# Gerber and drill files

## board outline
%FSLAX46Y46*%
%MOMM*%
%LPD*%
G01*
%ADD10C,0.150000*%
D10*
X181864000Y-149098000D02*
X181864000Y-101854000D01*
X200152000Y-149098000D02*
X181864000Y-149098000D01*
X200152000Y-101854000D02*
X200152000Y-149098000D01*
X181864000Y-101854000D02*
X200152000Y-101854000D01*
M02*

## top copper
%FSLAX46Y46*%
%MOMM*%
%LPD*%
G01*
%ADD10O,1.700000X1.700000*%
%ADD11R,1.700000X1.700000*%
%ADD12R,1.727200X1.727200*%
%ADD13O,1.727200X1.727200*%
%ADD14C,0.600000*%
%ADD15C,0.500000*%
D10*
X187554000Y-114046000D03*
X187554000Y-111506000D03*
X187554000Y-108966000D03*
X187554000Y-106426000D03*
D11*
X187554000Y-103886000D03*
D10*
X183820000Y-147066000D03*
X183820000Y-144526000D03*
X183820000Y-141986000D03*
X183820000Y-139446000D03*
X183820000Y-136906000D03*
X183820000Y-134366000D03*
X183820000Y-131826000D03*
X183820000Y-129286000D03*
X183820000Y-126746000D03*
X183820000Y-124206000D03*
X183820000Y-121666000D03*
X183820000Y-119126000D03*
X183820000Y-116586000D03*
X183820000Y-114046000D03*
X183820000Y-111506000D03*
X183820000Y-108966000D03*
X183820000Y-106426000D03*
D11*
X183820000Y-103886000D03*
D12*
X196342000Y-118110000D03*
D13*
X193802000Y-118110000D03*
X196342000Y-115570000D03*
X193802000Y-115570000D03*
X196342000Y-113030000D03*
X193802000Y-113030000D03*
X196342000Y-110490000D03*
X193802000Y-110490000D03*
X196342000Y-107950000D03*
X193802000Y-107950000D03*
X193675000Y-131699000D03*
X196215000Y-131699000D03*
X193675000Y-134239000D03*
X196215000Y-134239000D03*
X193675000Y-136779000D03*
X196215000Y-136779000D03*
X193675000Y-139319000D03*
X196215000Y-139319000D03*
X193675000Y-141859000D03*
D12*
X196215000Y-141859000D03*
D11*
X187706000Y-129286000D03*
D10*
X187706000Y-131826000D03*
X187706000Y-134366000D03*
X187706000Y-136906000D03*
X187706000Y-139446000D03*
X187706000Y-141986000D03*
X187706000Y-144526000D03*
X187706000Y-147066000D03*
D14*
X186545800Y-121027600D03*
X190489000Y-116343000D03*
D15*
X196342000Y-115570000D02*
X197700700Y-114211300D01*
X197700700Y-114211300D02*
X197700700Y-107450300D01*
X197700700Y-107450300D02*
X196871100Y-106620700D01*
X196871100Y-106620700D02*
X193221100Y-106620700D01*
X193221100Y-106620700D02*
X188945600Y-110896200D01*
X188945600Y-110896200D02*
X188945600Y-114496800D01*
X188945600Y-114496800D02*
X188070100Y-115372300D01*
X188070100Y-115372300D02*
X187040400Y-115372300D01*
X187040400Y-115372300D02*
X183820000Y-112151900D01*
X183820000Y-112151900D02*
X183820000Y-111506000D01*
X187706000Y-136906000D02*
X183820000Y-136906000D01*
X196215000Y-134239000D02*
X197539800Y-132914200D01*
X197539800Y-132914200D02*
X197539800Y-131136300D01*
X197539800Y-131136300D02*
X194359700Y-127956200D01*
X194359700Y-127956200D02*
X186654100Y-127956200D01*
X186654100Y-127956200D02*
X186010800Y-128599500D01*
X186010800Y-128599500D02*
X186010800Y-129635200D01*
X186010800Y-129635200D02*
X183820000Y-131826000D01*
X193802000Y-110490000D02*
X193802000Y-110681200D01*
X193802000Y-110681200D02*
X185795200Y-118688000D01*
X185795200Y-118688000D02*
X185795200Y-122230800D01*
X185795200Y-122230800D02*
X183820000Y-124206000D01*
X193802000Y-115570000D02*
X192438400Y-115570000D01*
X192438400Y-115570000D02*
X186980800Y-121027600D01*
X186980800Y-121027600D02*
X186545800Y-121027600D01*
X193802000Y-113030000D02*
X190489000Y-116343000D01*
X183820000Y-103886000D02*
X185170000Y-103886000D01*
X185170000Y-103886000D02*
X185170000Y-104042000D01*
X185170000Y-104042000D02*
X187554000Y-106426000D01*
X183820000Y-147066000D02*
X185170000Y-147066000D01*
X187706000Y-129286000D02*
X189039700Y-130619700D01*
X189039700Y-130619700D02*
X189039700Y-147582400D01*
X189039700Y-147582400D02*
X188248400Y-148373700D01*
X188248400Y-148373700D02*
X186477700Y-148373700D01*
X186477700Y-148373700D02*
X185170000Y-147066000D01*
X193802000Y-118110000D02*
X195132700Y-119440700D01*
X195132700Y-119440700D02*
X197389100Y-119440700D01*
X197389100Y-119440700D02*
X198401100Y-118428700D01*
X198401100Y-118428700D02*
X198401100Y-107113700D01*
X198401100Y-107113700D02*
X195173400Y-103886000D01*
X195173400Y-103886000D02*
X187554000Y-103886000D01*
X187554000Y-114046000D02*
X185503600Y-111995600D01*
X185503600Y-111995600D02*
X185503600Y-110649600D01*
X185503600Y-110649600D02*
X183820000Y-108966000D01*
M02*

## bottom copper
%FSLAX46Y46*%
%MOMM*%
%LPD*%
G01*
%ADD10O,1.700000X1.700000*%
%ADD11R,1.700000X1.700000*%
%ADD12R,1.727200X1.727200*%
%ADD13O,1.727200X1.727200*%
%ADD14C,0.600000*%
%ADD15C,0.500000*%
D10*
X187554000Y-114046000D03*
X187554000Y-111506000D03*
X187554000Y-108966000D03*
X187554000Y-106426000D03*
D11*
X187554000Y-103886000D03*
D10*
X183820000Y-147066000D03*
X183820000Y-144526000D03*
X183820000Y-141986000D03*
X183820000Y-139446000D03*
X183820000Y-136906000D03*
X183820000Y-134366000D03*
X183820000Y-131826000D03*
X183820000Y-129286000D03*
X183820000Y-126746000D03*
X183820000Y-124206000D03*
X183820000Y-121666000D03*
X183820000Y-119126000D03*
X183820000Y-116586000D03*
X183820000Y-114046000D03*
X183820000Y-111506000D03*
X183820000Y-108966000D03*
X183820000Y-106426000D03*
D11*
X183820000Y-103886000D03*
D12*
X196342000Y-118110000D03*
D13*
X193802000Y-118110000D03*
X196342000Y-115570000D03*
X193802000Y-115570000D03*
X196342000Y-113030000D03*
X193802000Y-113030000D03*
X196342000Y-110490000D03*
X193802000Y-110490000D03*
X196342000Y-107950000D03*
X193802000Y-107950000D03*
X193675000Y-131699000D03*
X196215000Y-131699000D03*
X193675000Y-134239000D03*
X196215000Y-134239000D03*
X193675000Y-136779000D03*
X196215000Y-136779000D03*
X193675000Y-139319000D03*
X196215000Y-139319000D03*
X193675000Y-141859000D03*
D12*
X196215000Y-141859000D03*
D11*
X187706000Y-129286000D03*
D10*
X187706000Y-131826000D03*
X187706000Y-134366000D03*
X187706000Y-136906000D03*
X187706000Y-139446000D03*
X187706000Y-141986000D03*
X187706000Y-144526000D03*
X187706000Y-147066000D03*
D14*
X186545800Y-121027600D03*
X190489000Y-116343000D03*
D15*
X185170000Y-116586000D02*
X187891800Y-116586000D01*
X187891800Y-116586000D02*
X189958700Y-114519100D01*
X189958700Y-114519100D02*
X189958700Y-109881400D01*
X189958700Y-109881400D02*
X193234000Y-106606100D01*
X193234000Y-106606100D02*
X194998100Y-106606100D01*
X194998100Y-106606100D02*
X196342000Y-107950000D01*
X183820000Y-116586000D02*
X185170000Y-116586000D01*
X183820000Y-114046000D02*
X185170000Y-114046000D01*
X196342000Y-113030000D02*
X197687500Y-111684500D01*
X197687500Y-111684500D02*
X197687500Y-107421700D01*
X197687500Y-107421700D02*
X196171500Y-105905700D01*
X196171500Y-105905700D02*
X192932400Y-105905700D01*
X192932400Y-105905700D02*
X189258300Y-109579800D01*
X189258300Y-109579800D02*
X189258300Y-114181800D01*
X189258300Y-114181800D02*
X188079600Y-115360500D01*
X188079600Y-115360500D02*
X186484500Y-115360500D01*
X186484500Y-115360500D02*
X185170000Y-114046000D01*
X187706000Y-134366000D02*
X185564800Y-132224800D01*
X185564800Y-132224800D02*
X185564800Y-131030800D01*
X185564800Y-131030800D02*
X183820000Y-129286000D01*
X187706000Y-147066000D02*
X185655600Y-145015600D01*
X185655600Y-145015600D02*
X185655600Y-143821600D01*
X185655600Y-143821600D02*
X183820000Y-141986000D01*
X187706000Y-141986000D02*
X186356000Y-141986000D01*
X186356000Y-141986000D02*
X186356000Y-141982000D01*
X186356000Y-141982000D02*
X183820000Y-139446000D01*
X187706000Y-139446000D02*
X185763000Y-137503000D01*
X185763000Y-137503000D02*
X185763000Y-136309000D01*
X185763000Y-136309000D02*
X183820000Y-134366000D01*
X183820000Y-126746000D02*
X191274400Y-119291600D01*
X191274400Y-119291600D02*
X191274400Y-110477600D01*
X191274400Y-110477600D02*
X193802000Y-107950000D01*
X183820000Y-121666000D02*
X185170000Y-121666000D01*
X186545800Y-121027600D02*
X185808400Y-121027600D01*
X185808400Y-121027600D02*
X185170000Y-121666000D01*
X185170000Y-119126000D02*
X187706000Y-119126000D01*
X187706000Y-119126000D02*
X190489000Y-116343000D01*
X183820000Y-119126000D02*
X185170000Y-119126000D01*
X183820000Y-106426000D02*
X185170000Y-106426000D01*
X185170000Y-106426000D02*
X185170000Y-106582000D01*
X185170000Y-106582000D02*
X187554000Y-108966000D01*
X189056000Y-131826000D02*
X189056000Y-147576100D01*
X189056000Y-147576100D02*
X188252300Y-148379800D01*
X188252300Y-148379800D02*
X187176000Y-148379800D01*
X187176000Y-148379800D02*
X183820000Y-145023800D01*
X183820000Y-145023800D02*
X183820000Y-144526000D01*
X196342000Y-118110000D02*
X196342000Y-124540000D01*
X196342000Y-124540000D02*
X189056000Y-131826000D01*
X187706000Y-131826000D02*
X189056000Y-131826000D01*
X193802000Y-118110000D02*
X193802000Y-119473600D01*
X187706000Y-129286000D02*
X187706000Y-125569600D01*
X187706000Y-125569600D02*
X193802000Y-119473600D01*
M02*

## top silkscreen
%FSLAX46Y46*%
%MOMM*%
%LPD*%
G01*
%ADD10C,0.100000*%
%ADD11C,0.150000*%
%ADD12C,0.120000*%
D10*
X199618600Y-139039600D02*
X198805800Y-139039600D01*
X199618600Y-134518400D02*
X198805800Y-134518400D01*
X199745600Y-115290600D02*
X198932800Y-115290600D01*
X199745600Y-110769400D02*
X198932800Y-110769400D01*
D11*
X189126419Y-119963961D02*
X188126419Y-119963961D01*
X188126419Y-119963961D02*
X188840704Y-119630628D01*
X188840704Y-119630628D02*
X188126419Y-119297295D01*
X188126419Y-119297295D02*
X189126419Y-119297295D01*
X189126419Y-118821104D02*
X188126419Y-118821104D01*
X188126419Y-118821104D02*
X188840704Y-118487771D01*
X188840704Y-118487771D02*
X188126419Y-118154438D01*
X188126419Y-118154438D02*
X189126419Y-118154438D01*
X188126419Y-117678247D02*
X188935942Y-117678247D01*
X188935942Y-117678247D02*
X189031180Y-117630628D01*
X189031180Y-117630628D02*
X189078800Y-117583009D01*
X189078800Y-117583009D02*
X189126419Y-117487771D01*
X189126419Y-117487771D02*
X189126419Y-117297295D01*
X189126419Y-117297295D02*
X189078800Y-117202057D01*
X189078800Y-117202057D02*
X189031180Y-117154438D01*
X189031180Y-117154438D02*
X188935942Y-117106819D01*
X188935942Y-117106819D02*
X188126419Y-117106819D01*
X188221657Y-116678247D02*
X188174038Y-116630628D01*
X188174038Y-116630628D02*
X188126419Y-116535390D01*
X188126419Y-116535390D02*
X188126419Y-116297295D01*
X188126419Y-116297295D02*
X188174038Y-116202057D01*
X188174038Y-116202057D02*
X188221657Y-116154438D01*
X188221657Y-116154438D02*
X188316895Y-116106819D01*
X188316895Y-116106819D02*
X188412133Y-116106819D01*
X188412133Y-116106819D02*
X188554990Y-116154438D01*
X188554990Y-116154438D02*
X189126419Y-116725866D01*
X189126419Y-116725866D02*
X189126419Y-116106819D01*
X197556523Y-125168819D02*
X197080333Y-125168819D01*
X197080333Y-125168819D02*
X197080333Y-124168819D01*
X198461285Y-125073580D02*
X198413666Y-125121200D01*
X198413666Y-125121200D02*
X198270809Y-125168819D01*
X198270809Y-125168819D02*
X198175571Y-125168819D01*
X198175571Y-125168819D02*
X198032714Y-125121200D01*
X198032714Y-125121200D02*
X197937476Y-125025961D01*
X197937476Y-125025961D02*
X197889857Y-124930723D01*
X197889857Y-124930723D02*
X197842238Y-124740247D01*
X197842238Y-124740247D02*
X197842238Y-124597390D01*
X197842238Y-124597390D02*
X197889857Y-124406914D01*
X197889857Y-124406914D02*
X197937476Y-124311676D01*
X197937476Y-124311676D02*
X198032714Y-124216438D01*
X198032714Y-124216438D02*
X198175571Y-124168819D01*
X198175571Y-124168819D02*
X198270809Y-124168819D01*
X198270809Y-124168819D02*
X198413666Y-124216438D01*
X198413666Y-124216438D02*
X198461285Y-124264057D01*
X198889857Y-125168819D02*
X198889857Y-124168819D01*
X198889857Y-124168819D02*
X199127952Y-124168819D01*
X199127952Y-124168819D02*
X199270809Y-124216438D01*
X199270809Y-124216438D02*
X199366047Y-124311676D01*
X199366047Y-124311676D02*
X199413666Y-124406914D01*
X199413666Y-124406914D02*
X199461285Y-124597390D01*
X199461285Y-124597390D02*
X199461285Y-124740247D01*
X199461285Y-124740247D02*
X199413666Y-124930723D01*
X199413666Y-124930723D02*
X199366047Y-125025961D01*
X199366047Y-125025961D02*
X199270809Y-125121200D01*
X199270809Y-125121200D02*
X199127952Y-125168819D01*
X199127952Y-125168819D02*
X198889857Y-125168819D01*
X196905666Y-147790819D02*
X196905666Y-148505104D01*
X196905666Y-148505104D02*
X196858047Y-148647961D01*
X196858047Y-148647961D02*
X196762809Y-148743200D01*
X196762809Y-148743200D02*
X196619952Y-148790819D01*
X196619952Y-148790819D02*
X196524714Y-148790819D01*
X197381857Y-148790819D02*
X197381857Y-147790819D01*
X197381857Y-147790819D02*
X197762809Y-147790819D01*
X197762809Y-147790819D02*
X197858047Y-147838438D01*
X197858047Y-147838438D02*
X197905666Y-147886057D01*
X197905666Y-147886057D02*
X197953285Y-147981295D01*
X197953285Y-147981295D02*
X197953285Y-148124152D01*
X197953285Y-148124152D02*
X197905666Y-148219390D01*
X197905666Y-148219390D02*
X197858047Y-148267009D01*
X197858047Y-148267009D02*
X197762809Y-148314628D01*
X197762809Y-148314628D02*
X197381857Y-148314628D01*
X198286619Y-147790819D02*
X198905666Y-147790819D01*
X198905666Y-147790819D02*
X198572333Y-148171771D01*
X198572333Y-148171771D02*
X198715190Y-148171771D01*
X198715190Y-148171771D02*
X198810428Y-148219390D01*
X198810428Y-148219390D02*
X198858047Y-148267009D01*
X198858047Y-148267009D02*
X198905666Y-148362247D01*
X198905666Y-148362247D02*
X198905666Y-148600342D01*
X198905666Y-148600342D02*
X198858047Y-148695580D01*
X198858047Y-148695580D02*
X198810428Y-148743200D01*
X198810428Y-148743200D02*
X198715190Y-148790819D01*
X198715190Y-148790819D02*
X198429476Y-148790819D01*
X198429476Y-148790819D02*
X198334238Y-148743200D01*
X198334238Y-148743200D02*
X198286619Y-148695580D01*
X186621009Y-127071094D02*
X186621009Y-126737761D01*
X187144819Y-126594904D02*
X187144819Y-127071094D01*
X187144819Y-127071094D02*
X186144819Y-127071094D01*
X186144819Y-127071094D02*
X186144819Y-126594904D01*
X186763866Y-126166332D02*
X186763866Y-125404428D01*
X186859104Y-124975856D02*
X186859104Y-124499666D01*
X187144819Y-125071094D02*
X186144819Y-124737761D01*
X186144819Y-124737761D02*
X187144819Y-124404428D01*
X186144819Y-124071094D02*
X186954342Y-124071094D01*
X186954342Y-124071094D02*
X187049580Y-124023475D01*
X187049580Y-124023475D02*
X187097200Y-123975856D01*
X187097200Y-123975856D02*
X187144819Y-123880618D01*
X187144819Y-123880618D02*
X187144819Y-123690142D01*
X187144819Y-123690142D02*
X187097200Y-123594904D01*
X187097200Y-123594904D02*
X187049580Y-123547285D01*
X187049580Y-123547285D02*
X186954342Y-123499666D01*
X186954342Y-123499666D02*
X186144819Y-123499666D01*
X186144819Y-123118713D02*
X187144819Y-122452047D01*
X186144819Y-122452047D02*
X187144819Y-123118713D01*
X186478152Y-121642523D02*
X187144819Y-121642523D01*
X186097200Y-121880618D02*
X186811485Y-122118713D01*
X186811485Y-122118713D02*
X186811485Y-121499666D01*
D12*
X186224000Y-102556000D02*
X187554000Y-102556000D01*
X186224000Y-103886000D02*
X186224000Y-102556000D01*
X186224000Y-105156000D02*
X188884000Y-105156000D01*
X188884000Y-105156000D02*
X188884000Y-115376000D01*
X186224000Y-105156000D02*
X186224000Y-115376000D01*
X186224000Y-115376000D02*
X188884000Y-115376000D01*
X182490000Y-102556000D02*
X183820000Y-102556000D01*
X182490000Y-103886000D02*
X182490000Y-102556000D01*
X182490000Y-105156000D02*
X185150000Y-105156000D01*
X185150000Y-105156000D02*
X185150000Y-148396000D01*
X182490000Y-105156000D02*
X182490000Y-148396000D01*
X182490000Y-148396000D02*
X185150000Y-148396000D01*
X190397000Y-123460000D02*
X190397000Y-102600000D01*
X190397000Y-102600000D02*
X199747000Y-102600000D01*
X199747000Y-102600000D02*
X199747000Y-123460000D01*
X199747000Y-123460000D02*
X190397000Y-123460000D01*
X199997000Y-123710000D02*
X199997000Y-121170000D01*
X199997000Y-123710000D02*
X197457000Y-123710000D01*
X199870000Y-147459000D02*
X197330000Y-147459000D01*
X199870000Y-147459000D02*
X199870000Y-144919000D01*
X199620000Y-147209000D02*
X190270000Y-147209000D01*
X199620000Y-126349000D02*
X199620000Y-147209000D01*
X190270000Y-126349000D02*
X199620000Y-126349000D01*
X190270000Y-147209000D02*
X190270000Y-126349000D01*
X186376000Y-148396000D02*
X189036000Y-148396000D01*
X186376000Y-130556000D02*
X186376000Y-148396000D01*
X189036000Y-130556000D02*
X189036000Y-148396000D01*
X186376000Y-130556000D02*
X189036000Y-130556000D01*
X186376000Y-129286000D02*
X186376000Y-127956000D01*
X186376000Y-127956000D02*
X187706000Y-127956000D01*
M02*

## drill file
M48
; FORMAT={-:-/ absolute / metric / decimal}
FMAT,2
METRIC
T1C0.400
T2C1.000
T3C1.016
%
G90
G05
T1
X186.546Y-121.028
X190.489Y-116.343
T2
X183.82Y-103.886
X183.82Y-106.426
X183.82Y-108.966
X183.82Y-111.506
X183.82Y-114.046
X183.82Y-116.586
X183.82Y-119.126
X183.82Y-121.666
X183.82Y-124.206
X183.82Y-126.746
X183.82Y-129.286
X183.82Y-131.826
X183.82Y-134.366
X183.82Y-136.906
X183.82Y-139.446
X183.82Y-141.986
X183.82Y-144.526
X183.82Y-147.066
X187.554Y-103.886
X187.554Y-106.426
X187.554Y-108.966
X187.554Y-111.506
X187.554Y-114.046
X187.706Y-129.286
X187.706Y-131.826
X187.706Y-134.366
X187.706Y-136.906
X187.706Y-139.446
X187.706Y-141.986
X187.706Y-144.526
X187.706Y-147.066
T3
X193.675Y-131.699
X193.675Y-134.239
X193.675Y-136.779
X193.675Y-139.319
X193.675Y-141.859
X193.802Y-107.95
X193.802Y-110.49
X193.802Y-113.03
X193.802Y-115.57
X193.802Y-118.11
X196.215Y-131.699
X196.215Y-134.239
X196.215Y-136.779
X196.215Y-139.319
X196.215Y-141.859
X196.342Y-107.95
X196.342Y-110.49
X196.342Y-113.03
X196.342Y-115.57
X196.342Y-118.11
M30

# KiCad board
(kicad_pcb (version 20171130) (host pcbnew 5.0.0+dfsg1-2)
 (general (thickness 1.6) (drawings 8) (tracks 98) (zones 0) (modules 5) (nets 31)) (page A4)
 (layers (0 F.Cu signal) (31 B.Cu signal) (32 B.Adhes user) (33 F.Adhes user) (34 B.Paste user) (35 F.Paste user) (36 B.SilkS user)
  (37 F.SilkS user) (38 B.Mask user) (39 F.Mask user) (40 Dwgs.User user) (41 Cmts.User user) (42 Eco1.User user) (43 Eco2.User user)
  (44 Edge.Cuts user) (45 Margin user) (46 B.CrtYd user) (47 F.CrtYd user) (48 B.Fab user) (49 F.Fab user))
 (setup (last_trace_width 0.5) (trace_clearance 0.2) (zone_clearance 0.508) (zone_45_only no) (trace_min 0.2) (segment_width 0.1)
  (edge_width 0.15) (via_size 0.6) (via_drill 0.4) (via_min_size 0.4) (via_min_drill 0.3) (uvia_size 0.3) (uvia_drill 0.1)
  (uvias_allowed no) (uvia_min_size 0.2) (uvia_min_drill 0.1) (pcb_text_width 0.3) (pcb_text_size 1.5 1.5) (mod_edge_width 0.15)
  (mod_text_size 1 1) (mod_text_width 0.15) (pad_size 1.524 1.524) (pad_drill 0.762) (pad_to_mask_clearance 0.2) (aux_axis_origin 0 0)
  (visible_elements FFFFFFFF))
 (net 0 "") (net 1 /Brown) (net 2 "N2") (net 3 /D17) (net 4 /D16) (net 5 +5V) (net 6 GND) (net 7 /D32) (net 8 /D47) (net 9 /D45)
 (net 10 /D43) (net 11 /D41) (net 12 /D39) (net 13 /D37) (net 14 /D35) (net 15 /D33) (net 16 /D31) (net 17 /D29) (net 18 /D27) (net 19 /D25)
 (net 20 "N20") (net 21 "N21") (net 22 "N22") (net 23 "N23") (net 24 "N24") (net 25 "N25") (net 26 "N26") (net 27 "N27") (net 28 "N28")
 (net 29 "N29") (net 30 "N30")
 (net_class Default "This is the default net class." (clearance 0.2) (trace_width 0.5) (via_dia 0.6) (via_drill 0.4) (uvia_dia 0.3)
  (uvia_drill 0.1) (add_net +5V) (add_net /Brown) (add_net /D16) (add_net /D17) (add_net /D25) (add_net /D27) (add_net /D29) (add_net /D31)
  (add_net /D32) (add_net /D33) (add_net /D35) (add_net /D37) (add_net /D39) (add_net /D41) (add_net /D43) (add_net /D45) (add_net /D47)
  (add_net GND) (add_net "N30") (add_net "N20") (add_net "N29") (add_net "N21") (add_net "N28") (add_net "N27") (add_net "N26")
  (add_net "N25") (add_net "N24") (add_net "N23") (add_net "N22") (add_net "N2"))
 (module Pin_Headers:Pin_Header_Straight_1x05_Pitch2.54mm (layer F.Cu) (at 187.554 103.886)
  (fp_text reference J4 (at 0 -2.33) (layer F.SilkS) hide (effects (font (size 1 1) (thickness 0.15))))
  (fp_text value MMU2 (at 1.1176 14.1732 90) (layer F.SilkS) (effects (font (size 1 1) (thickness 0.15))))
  (fp_line (start -1.33 -1.33) (end 0 -1.33) (layer F.SilkS) (width 0.12))
  (fp_line (start -1.33 0) (end -1.33 -1.33) (layer F.SilkS) (width 0.12))
  (fp_line (start -1.33 1.27) (end 1.33 1.27) (layer F.SilkS) (width 0.12))
  (fp_line (start 1.33 1.27) (end 1.33 11.49) (layer F.SilkS) (width 0.12))
  (fp_line (start -1.33 1.27) (end -1.33 11.49) (layer F.SilkS) (width 0.12))
  (fp_line (start -1.33 11.49) (end 1.33 11.49) (layer F.SilkS) (width 0.12))
  (pad 5 thru_hole oval (at 0 10.16) (size 1.7 1.7) (drill 1) (layers *.Cu *.Mask) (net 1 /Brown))
  (pad 4 thru_hole oval (at 0 7.62) (size 1.7 1.7) (drill 1) (layers *.Cu *.Mask) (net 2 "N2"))
  (pad 3 thru_hole oval (at 0 5.08) (size 1.7 1.7) (drill 1) (layers *.Cu *.Mask) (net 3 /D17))
  (pad 2 thru_hole oval (at 0 2.54) (size 1.7 1.7) (drill 1) (layers *.Cu *.Mask) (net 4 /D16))
  (pad 1 thru_hole rect (at 0 0) (size 1.7 1.7) (drill 1) (layers *.Cu *.Mask) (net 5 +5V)))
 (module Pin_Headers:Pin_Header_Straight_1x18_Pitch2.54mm (layer F.Cu) (at 183.82 103.886)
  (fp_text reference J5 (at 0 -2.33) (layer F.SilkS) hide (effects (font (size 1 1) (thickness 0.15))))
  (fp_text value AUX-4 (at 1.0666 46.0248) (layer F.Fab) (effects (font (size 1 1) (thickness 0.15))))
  (fp_line (start -1.33 -1.33) (end 0 -1.33) (layer F.SilkS) (width 0.12))
  (fp_line (start -1.33 0) (end -1.33 -1.33) (layer F.SilkS) (width 0.12))
  (fp_line (start -1.33 1.27) (end 1.33 1.27) (layer F.SilkS) (width 0.12))
  (fp_line (start 1.33 1.27) (end 1.33 44.51) (layer F.SilkS) (width 0.12))
  (fp_line (start -1.33 1.27) (end -1.33 44.51) (layer F.SilkS) (width 0.12))
  (fp_line (start -1.33 44.51) (end 1.33 44.51) (layer F.SilkS) (width 0.12))
  (pad 18 thru_hole oval (at 0 43.18) (size 1.7 1.7) (drill 1) (layers *.Cu *.Mask) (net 5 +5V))
  (pad 17 thru_hole oval (at 0 40.64) (size 1.7 1.7) (drill 1) (layers *.Cu *.Mask) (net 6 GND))
  (pad 16 thru_hole oval (at 0 38.1) (size 1.7 1.7) (drill 1) (layers *.Cu *.Mask) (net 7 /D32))
  (pad 15 thru_hole oval (at 0 35.56) (size 1.7 1.7) (drill 1) (layers *.Cu *.Mask) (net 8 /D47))
  (pad 14 thru_hole oval (at 0 33.02) (size 1.7 1.7) (drill 1) (layers *.Cu *.Mask) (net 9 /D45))
  (pad 13 thru_hole oval (at 0 30.48) (size 1.7 1.7) (drill 1) (layers *.Cu *.Mask) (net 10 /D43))
  (pad 12 thru_hole oval (at 0 27.94) (size 1.7 1.7) (drill 1) (layers *.Cu *.Mask) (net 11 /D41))
  (pad 11 thru_hole oval (at 0 25.4) (size 1.7 1.7) (drill 1) (layers *.Cu *.Mask) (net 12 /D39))
  (pad 10 thru_hole oval (at 0 22.86) (size 1.7 1.7) (drill 1) (layers *.Cu *.Mask) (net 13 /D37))
  (pad 9 thru_hole oval (at 0 20.32) (size 1.7 1.7) (drill 1) (layers *.Cu *.Mask) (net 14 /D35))
  (pad 8 thru_hole oval (at 0 17.78) (size 1.7 1.7) (drill 1) (layers *.Cu *.Mask) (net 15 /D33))
  (pad 7 thru_hole oval (at 0 15.24) (size 1.7 1.7) (drill 1) (layers *.Cu *.Mask) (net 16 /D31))
  (pad 6 thru_hole oval (at 0 12.7) (size 1.7 1.7) (drill 1) (layers *.Cu *.Mask) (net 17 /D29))
  (pad 5 thru_hole oval (at 0 10.16) (size 1.7 1.7) (drill 1) (layers *.Cu *.Mask) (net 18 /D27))
  (pad 4 thru_hole oval (at 0 7.62) (size 1.7 1.7) (drill 1) (layers *.Cu *.Mask) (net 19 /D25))
  (pad 3 thru_hole oval (at 0 5.08) (size 1.7 1.7) (drill 1) (layers *.Cu *.Mask) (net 1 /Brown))
  (pad 2 thru_hole oval (at 0 2.54) (size 1.7 1.7) (drill 1) (layers *.Cu *.Mask) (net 3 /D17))
  (pad 1 thru_hole rect (at 0 0) (size 1.7 1.7) (drill 1) (layers *.Cu *.Mask) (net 4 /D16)))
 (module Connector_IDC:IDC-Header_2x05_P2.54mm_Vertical (layer F.Cu) (at 196.342 118.11 180)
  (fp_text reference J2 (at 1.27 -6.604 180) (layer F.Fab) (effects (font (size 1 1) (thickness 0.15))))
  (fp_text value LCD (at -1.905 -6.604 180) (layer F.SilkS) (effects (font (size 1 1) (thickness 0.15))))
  (fp_line (start 5.945 -5.35) (end 5.945 15.51) (layer F.SilkS) (width 0.12))
  (fp_line (start 5.945 15.51) (end -3.405 15.51) (layer F.SilkS) (width 0.12))
  (fp_line (start -3.405 15.51) (end -3.405 -5.35) (layer F.SilkS) (width 0.12))
  (fp_line (start -3.405 -5.35) (end 5.945 -5.35) (layer F.SilkS) (width 0.12))
  (fp_line (start -3.655 -5.6) (end -3.655 -3.06) (layer F.SilkS) (width 0.12))
  (fp_line (start -3.655 -5.6) (end -1.115 -5.6) (layer F.SilkS) (width 0.12))
  (pad 1 thru_hole rect (at 0 0 180) (size 1.7272 1.7272) (drill 1.016) (layers *.Cu *.Mask) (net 6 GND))
  (pad 2 thru_hole oval (at 2.54 0 180) (size 1.7272 1.7272) (drill 1.016) (layers *.Cu *.Mask) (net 5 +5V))
  (pad 3 thru_hole oval (at 0 2.54 180) (size 1.7272 1.7272) (drill 1.016) (layers *.Cu *.Mask) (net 19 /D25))
  (pad 4 thru_hole oval (at 2.54 2.54 180) (size 1.7272 1.7272) (drill 1.016) (layers *.Cu *.Mask) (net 15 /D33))
  (pad 5 thru_hole oval (at 0 5.08 180) (size 1.7272 1.7272) (drill 1.016) (layers *.Cu *.Mask) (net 18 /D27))
  (pad 6 thru_hole oval (at 2.54 5.08 180) (size 1.7272 1.7272) (drill 1.016) (layers *.Cu *.Mask) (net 16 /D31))
  (pad 7 thru_hole oval (at 0 7.62 180) (size 1.7272 1.7272) (drill 1.016) (layers *.Cu *.Mask) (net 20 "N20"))
  (pad 8 thru_hole oval (at 2.54 7.62 180) (size 1.7272 1.7272) (drill 1.016) (layers *.Cu *.Mask) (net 14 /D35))
  (pad 9 thru_hole oval (at 0 10.16 180) (size 1.7272 1.7272) (drill 1.016) (layers *.Cu *.Mask) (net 17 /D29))
  (pad 10 thru_hole oval (at 2.54 10.16 180) (size 1.7272 1.7272) (drill 1.016) (layers *.Cu *.Mask) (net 13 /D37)))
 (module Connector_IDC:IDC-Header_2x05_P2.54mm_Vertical (layer F.Cu) (at 196.215 141.859 180)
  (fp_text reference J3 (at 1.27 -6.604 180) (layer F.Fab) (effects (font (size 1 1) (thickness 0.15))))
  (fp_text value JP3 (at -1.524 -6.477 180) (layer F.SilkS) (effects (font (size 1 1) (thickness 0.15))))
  (fp_line (start -3.655 -5.6) (end -1.115 -5.6) (layer F.SilkS) (width 0.12))
  (fp_line (start -3.655 -5.6) (end -3.655 -3.06) (layer F.SilkS) (width 0.12))
  (fp_line (start -3.405 -5.35) (end 5.945 -5.35) (layer F.SilkS) (width 0.12))
  (fp_line (start -3.405 15.51) (end -3.405 -5.35) (layer F.SilkS) (width 0.12))
  (fp_line (start 5.945 15.51) (end -3.405 15.51) (layer F.SilkS) (width 0.12))
  (fp_line (start 5.945 -5.35) (end 5.945 15.51) (layer F.SilkS) (width 0.12))
  (pad 10 thru_hole oval (at 2.54 10.16 180) (size 1.7272 1.7272) (drill 1.016) (layers *.Cu *.Mask) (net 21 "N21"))
  (pad 9 thru_hole oval (at 0 10.16 180) (size 1.7272 1.7272) (drill 1.016) (layers *.Cu *.Mask) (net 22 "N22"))
  (pad 8 thru_hole oval (at 2.54 7.62 180) (size 1.7272 1.7272) (drill 1.016) (layers *.Cu *.Mask) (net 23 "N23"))
  (pad 7 thru_hole oval (at 0 7.62 180) (size 1.7272 1.7272) (drill 1.016) (layers *.Cu *.Mask) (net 11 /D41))
  (pad 6 thru_hole oval (at 2.54 5.08 180) (size 1.7272 1.7272) (drill 1.016) (layers *.Cu *.Mask) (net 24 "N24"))
  (pad 5 thru_hole oval (at 0 5.08 180) (size 1.7272 1.7272) (drill 1.016) (layers *.Cu *.Mask) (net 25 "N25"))
  (pad 4 thru_hole oval (at 2.54 2.54 180) (size 1.7272 1.7272) (drill 1.016) (layers *.Cu *.Mask) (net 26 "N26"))
  (pad 3 thru_hole oval (at 0 2.54 180) (size 1.7272 1.7272) (drill 1.016) (layers *.Cu *.Mask) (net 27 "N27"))
  (pad 2 thru_hole oval (at 2.54 0 180) (size 1.7272 1.7272) (drill 1.016) (layers *.Cu *.Mask) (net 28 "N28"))
  (pad 1 thru_hole rect (at 0 0 180) (size 1.7272 1.7272) (drill 1.016) (layers *.Cu *.Mask) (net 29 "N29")))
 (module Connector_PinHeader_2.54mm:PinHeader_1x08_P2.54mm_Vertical (layer F.Cu) (at 187.706 129.286)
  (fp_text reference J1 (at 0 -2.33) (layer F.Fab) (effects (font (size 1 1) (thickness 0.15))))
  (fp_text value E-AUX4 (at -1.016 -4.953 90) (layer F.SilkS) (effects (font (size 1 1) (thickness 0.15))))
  (fp_line (start -1.33 19.11) (end 1.33 19.11) (layer F.SilkS) (width 0.12))
  (fp_line (start -1.33 1.27) (end -1.33 19.11) (layer F.SilkS) (width 0.12))
  (fp_line (start 1.33 1.27) (end 1.33 19.11) (layer F.SilkS) (width 0.12))
  (fp_line (start -1.33 1.27) (end 1.33 1.27) (layer F.SilkS) (width 0.12))
  (fp_line (start -1.33 0) (end -1.33 -1.33) (layer F.SilkS) (width 0.12))
  (fp_line (start -1.33 -1.33) (end 0 -1.33) (layer F.SilkS) (width 0.12))
  (pad 1 thru_hole rect (at 0 0) (size 1.7 1.7) (drill 1) (layers *.Cu *.Mask) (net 5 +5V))
  (pad 2 thru_hole oval (at 0 2.54) (size 1.7 1.7) (drill 1) (layers *.Cu *.Mask) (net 6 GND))
  (pad 3 thru_hole oval (at 0 5.08) (size 1.7 1.7) (drill 1) (layers *.Cu *.Mask) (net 12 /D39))
  (pad 4 thru_hole oval (at 0 7.62) (size 1.7 1.7) (drill 1) (layers *.Cu *.Mask) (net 9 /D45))
  (pad 5 thru_hole oval (at 0 10.16) (size 1.7 1.7) (drill 1) (layers *.Cu *.Mask) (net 10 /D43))
  (pad 6 thru_hole oval (at 0 12.7) (size 1.7 1.7) (drill 1) (layers *.Cu *.Mask) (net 8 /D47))
  (pad 7 thru_hole oval (at 0 15.24) (size 1.7 1.7) (drill 1) (layers *.Cu *.Mask) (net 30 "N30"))
  (pad 8 thru_hole oval (at 0 17.78) (size 1.7 1.7) (drill 1) (layers *.Cu *.Mask) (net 7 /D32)))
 (gr_line (start 199.6186 139.0396) (end 198.8058 139.0396) (layer F.SilkS) (width 0.1))
 (gr_line (start 199.6186 134.5184) (end 198.8058 134.5184) (layer F.SilkS) (width 0.1))
 (gr_line (start 199.7456 115.2906) (end 198.9328 115.2906) (layer F.SilkS) (width 0.1))
 (gr_line (start 199.7456 110.7694) (end 198.9328 110.7694) (layer F.SilkS) (width 0.1))
 (gr_line (start 181.864 149.098) (end 181.864 101.854) (layer Edge.Cuts) (width 0.15))
 (gr_line (start 200.152 149.098) (end 181.864 149.098) (layer Edge.Cuts) (width 0.15))
 (gr_line (start 200.152 101.854) (end 200.152 149.098) (layer Edge.Cuts) (width 0.15))
 (gr_line (start 181.864 101.854) (end 200.152 101.854) (layer Edge.Cuts) (width 0.15))
 (segment (start 185.17 116.586) (end 187.8918 116.586) (width 0.5) (layer B.Cu) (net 17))
 (segment (start 187.8918 116.586) (end 189.9587 114.5191) (width 0.5) (layer B.Cu) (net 17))
 (segment (start 189.9587 114.5191) (end 189.9587 109.8814) (width 0.5) (layer B.Cu) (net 17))
 (segment (start 189.9587 109.8814) (end 193.234 106.6061) (width 0.5) (layer B.Cu) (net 17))
 (segment (start 193.234 106.6061) (end 194.9981 106.6061) (width 0.5) (layer B.Cu) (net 17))
 (segment (start 194.9981 106.6061) (end 196.342 107.95) (width 0.5) (layer B.Cu) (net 17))
 (segment (start 183.82 116.586) (end 185.17 116.586) (width 0.5) (layer B.Cu) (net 17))
 (segment (start 183.82 114.046) (end 185.17 114.046) (width 0.5) (layer B.Cu) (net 18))
 (segment (start 196.342 113.03) (end 197.6875 111.6845) (width 0.5) (layer B.Cu) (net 18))
 (segment (start 197.6875 111.6845) (end 197.6875 107.4217) (width 0.5) (layer B.Cu) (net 18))
 (segment (start 197.6875 107.4217) (end 196.1715 105.9057) (width 0.5) (layer B.Cu) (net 18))
 (segment (start 196.1715 105.9057) (end 192.9324 105.9057) (width 0.5) (layer B.Cu) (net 18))
 (segment (start 192.9324 105.9057) (end 189.2583 109.5798) (width 0.5) (layer B.Cu) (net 18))
 (segment (start 189.2583 109.5798) (end 189.2583 114.1818) (width 0.5) (layer B.Cu) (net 18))
 (segment (start 189.2583 114.1818) (end 188.0796 115.3605) (width 0.5) (layer B.Cu) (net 18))
 (segment (start 188.0796 115.3605) (end 186.4845 115.3605) (width 0.5) (layer B.Cu) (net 18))
 (segment (start 186.4845 115.3605) (end 185.17 114.046) (width 0.5) (layer B.Cu) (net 18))
 (segment (start 196.342 115.57) (end 197.7007 114.2113) (width 0.5) (layer F.Cu) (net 19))
 (segment (start 197.7007 114.2113) (end 197.7007 107.4503) (width 0.5) (layer F.Cu) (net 19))
 (segment (start 197.7007 107.4503) (end 196.8711 106.6207) (width 0.5) (layer F.Cu) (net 19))
 (segment (start 196.8711 106.6207) (end 193.2211 106.6207) (width 0.5) (layer F.Cu) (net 19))
 (segment (start 193.2211 106.6207) (end 188.9456 110.8962) (width 0.5) (layer F.Cu) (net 19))
 (segment (start 188.9456 110.8962) (end 188.9456 114.4968) (width 0.5) (layer F.Cu) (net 19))
 (segment (start 188.9456 114.4968) (end 188.0701 115.3723) (width 0.5) (layer F.Cu) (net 19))
 (segment (start 188.0701 115.3723) (end 187.0404 115.3723) (width 0.5) (layer F.Cu) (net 19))
 (segment (start 187.0404 115.3723) (end 183.82 112.1519) (width 0.5) (layer F.Cu) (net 19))
 (segment (start 183.82 112.1519) (end 183.82 111.506) (width 0.5) (layer F.Cu) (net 19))
 (segment (start 187.706 134.366) (end 185.5648 132.2248) (width 0.5) (layer B.Cu) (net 12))
 (segment (start 185.5648 132.2248) (end 185.5648 131.0308) (width 0.5) (layer B.Cu) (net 12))
 (segment (start 185.5648 131.0308) (end 183.82 129.286) (width 0.5) (layer B.Cu) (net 12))
 (segment (start 187.706 147.066) (end 185.6556 145.0156) (width 0.5) (layer B.Cu) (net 7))
 (segment (start 185.6556 145.0156) (end 185.6556 143.8216) (width 0.5) (layer B.Cu) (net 7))
 (segment (start 185.6556 143.8216) (end 183.82 141.986) (width 0.5) (layer B.Cu) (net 7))
 (segment (start 187.706 141.986) (end 186.356 141.986) (width 0.5) (layer B.Cu) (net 8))
 (segment (start 186.356 141.986) (end 186.356 141.982) (width 0.5) (layer B.Cu) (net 8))
 (segment (start 186.356 141.982) (end 183.82 139.446) (width 0.5) (layer B.Cu) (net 8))
 (segment (start 187.706 136.906) (end 183.82 136.906) (width 0.5) (layer F.Cu) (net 9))
 (segment (start 187.706 139.446) (end 185.763 137.503) (width 0.5) (layer B.Cu) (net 10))
 (segment (start 185.763 137.503) (end 185.763 136.309) (width 0.5) (layer B.Cu) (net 10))
 (segment (start 185.763 136.309) (end 183.82 134.366) (width 0.5) (layer B.Cu) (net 10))
 (segment (start 196.215 134.239) (end 197.5398 132.9142) (width 0.5) (layer F.Cu) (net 11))
 (segment (start 197.5398 132.9142) (end 197.5398 131.1363) (width 0.5) (layer F.Cu) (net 11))
 (segment (start 197.5398 131.1363) (end 194.3597 127.9562) (width 0.5) (layer F.Cu) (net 11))
 (segment (start 194.3597 127.9562) (end 186.6541 127.9562) (width 0.5) (layer F.Cu) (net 11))
 (segment (start 186.6541 127.9562) (end 186.0108 128.5995) (width 0.5) (layer F.Cu) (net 11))
 (segment (start 186.0108 128.5995) (end 186.0108 129.6352) (width 0.5) (layer F.Cu) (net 11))
 (segment (start 186.0108 129.6352) (end 183.82 131.826) (width 0.5) (layer F.Cu) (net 11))
 (segment (start 183.82 126.746) (end 191.2744 119.2916) (width 0.5) (layer B.Cu) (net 13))
 (segment (start 191.2744 119.2916) (end 191.2744 110.4776) (width 0.5) (layer B.Cu) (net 13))
 (segment (start 191.2744 110.4776) (end 193.802 107.95) (width 0.5) (layer B.Cu) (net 13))
 (segment (start 193.802 110.49) (end 193.802 110.6812) (width 0.5) (layer F.Cu) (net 14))
 (segment (start 193.802 110.6812) (end 185.7952 118.688) (width 0.5) (layer F.Cu) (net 14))
 (segment (start 185.7952 118.688) (end 185.7952 122.2308) (width 0.5) (layer F.Cu) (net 14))
 (segment (start 185.7952 122.2308) (end 183.82 124.206) (width 0.5) (layer F.Cu) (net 14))
 (segment (start 183.82 121.666) (end 185.17 121.666) (width 0.5) (layer B.Cu) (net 15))
 (segment (start 193.802 115.57) (end 192.4384 115.57) (width 0.5) (layer F.Cu) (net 15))
 (segment (start 186.5458 121.0276) (end 185.8084 121.0276) (width 0.5) (layer B.Cu) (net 15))
 (segment (start 185.8084 121.0276) (end 185.17 121.666) (width 0.5) (layer B.Cu) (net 15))
 (segment (start 192.4384 115.57) (end 186.9808 121.0276) (width 0.5) (layer F.Cu) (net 15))
 (segment (start 186.9808 121.0276) (end 186.5458 121.0276) (width 0.5) (layer F.Cu) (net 15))
 (via (at 186.5458 121.0276) (size 0.6) (layers F.Cu B.Cu) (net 15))
 (segment (start 193.802 113.03) (end 190.489 116.343) (width 0.5) (layer F.Cu) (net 16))
 (segment (start 185.17 119.126) (end 187.706 119.126) (width 0.5) (layer B.Cu) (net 16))
 (segment (start 187.706 119.126) (end 190.489 116.343) (width 0.5) (layer B.Cu) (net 16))
 (segment (start 183.82 119.126) (end 185.17 119.126) (width 0.5) (layer B.Cu) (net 16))
 (via (at 190.489 116.343) (size 0.6) (layers F.Cu B.Cu) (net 16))
 (segment (start 183.82 106.426) (end 185.17 106.426) (width 0.5) (layer B.Cu) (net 3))
 (segment (start 185.17 106.426) (end 185.17 106.582) (width 0.5) (layer B.Cu) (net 3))
 (segment (start 185.17 106.582) (end 187.554 108.966) (width 0.5) (layer B.Cu) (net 3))
 (segment (start 183.82 103.886) (end 185.17 103.886) (width 0.5) (layer F.Cu) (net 4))
 (segment (start 185.17 103.886) (end 185.17 104.042) (width 0.5) (layer F.Cu) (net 4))
 (segment (start 185.17 104.042) (end 187.554 106.426) (width 0.5) (layer F.Cu) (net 4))
 (segment (start 189.056 131.826) (end 189.056 147.5761) (width 0.5) (layer B.Cu) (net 6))
 (segment (start 189.056 147.5761) (end 188.2523 148.3798) (width 0.5) (layer B.Cu) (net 6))
 (segment (start 188.2523 148.3798) (end 187.176 148.3798) (width 0.5) (layer B.Cu) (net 6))
 (segment (start 187.176 148.3798) (end 183.82 145.0238) (width 0.5) (layer B.Cu) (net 6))
 (segment (start 183.82 145.0238) (end 183.82 144.526) (width 0.5) (layer B.Cu) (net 6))
 (segment (start 196.342 118.11) (end 196.342 124.54) (width 0.5) (layer B.Cu) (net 6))
 (segment (start 196.342 124.54) (end 189.056 131.826) (width 0.5) (layer B.Cu) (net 6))
 (segment (start 187.706 131.826) (end 189.056 131.826) (width 0.5) (layer B.Cu) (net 6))
 (segment (start 183.82 147.066) (end 185.17 147.066) (width 0.5) (layer F.Cu) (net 5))
 (segment (start 187.706 129.286) (end 189.0397 130.6197) (width 0.5) (layer F.Cu) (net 5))
 (segment (start 189.0397 130.6197) (end 189.0397 147.5824) (width 0.5) (layer F.Cu) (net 5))
 (segment (start 189.0397 147.5824) (end 188.2484 148.3737) (width 0.5) (layer F.Cu) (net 5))
 (segment (start 188.2484 148.3737) (end 186.4777 148.3737) (width 0.5) (layer F.Cu) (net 5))
 (segment (start 186.4777 148.3737) (end 185.17 147.066) (width 0.5) (layer F.Cu) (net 5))
 (segment (start 193.802 118.11) (end 193.802 119.4736) (width 0.5) (layer B.Cu) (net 5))
 (segment (start 187.706 129.286) (end 187.706 125.5696) (width 0.5) (layer B.Cu) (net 5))
 (segment (start 187.706 125.5696) (end 193.802 119.4736) (width 0.5) (layer B.Cu) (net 5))
 (segment (start 193.802 118.11) (end 195.1327 119.4407) (width 0.5) (layer F.Cu) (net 5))
 (segment (start 195.1327 119.4407) (end 197.3891 119.4407) (width 0.5) (layer F.Cu) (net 5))
 (segment (start 197.3891 119.4407) (end 198.4011 118.4287) (width 0.5) (layer F.Cu) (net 5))
 (segment (start 198.4011 118.4287) (end 198.4011 107.1137) (width 0.5) (layer F.Cu) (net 5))
 (segment (start 198.4011 107.1137) (end 195.1734 103.886) (width 0.5) (layer F.Cu) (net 5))
 (segment (start 195.1734 103.886) (end 187.554 103.886) (width 0.5) (layer F.Cu) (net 5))
 (segment (start 187.554 114.046) (end 185.5036 111.9956) (width 0.5) (layer F.Cu) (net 1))
 (segment (start 185.5036 111.9956) (end 185.5036 110.6496) (width 0.5) (layer F.Cu) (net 1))
 (segment (start 185.5036 110.6496) (end 183.82 108.966) (width 0.5) (layer F.Cu) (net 1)))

